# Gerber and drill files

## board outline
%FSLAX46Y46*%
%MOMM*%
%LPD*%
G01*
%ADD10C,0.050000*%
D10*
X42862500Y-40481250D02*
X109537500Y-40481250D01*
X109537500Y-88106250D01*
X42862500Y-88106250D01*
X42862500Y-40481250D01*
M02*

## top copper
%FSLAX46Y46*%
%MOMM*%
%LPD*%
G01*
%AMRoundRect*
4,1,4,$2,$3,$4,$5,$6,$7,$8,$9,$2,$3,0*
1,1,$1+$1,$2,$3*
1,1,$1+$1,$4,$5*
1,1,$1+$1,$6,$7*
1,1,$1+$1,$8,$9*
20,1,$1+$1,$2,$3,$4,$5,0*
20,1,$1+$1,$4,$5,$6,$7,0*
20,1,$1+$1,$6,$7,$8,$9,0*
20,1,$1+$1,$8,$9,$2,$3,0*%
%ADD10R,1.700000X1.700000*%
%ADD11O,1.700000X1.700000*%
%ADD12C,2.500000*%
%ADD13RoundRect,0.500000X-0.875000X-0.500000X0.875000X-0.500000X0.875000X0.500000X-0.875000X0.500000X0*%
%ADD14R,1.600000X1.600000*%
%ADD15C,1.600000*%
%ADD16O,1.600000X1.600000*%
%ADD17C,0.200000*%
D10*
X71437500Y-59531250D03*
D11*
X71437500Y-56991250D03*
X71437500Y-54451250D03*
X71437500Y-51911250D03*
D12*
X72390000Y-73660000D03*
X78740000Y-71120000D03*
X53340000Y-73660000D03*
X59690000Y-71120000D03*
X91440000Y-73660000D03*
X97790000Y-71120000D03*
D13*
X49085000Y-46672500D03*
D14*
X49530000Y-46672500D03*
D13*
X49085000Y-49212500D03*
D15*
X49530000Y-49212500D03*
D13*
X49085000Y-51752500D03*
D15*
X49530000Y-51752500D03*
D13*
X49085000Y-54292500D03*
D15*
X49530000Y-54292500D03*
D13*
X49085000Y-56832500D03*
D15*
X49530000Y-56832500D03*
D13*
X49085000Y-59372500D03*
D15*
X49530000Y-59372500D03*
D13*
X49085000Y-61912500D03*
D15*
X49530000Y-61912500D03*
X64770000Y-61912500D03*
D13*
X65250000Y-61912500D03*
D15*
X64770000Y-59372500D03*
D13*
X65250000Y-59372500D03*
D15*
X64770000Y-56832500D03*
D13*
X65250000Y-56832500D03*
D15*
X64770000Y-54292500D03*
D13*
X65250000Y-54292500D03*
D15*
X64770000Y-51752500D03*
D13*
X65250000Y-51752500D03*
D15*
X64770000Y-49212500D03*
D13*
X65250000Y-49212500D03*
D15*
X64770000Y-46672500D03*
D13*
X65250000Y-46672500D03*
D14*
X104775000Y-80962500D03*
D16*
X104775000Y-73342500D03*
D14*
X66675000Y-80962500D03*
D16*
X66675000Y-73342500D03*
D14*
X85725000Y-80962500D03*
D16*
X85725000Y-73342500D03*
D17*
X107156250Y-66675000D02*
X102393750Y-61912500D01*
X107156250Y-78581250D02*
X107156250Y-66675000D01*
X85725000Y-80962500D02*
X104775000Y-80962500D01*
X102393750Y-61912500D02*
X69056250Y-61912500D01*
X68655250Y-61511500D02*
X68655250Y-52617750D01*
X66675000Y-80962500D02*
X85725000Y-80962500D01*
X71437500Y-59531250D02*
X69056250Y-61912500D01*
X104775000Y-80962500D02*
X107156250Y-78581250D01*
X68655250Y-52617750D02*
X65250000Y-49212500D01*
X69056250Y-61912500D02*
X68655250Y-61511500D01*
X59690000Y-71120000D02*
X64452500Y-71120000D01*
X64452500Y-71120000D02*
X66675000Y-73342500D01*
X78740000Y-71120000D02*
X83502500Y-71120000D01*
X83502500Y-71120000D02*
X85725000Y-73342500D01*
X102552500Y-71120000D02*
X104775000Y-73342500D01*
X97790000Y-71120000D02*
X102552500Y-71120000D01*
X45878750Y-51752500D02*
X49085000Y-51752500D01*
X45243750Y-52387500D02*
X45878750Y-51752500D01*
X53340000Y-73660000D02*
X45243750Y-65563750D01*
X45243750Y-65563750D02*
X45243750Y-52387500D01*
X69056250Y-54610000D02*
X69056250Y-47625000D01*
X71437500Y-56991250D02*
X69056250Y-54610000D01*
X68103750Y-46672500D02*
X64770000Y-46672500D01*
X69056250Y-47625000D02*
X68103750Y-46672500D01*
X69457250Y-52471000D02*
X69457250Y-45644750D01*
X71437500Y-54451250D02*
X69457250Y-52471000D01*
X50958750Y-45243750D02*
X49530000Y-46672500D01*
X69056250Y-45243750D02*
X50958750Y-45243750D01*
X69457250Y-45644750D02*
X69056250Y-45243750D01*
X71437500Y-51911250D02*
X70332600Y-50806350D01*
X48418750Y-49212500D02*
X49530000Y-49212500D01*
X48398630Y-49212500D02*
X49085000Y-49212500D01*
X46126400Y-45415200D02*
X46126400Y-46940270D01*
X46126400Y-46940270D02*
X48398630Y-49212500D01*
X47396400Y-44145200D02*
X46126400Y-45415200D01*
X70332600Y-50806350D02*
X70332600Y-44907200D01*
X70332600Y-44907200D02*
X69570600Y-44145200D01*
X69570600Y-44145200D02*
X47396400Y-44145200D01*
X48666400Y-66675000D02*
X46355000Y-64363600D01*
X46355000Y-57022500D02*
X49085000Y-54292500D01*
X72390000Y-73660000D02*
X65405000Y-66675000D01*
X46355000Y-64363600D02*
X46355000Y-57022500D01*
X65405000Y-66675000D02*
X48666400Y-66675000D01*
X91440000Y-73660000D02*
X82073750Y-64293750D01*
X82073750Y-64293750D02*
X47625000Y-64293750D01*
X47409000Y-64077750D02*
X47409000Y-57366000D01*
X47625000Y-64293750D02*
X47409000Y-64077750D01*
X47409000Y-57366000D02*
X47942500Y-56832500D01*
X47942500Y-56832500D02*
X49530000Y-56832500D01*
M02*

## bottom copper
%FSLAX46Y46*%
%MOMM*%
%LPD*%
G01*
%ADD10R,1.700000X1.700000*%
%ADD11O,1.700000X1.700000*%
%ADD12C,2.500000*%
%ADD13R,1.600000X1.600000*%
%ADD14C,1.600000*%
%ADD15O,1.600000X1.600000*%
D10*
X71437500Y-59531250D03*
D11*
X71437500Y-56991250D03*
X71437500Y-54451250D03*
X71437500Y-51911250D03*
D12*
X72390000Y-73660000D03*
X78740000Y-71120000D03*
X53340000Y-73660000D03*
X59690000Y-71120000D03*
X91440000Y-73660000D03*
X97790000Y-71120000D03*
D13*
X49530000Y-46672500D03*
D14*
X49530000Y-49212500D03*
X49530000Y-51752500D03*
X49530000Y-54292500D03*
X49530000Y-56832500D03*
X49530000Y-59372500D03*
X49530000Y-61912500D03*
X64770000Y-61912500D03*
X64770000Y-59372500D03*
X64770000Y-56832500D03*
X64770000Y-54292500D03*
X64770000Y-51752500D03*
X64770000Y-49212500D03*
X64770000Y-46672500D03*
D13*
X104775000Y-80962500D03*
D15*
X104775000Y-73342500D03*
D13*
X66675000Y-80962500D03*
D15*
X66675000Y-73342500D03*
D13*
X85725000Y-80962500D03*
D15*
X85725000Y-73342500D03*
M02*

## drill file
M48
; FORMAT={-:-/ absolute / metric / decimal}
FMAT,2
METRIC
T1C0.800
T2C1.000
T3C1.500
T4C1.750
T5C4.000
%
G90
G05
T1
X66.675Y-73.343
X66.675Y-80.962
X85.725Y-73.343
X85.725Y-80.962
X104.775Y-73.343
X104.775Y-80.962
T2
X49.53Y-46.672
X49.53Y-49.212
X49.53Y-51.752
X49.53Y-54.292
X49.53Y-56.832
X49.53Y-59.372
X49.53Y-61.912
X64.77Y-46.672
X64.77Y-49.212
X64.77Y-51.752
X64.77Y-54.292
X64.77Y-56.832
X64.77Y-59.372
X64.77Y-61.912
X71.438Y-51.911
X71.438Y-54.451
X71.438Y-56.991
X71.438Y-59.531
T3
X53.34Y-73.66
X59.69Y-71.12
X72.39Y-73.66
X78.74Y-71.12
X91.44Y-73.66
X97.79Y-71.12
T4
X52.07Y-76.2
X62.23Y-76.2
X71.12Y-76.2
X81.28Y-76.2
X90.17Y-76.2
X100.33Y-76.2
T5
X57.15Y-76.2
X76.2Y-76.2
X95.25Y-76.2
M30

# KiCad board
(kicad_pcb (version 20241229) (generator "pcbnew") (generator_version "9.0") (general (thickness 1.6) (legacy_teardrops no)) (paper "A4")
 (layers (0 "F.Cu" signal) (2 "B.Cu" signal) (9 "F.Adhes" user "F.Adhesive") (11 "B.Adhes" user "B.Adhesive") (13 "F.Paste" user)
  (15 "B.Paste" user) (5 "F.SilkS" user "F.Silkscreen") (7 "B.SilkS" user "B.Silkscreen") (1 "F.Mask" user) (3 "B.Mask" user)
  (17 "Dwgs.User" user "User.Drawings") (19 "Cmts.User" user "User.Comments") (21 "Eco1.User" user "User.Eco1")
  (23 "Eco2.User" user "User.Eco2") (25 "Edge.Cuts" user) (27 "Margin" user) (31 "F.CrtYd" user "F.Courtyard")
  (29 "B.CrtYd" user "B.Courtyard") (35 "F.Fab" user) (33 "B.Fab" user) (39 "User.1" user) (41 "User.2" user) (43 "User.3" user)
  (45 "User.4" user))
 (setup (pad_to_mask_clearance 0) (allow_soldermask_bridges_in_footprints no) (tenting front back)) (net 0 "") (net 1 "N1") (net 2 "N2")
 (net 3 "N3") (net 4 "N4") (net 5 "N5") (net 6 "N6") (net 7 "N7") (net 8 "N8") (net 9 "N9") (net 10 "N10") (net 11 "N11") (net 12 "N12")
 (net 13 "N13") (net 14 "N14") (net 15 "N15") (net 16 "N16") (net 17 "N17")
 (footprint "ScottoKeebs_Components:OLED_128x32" (layer "F.Cu") (at 69.8375 49.73125)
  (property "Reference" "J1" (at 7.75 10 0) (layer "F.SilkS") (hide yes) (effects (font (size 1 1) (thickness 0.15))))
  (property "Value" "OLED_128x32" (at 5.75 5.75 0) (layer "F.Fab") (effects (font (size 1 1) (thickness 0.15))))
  (pad "1" thru_hole rect (at 1.6 9.8 180) (size 1.7 1.7) (drill 1) (layers "*.Cu" "*.Mask") (remove_unused_layers no) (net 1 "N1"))
  (pad "2" thru_hole oval (at 1.6 7.26 180) (size 1.7 1.7) (drill 1) (layers "*.Cu" "*.Mask") (remove_unused_layers no) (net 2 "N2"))
  (pad "3" thru_hole oval (at 1.6 4.72 180) (size 1.7 1.7) (drill 1) (layers "*.Cu" "*.Mask") (remove_unused_layers no) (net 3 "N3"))
  (pad "4" thru_hole oval (at 1.6 2.18 180) (size 1.7 1.7) (drill 1) (layers "*.Cu" "*.Mask") (remove_unused_layers no) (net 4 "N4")))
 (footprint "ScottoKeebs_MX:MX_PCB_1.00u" (layer "F.Cu") (at 76.2 76.2)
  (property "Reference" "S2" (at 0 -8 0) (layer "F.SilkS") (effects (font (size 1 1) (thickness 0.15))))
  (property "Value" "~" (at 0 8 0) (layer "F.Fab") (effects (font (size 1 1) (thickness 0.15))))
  (pad "" np_thru_hole circle (at -5.08 0) (size 1.75 1.75) (drill 1.75) (layers "*.Cu" "*.Mask"))
  (pad "" np_thru_hole circle (at 0 0) (size 4 4) (drill 4) (layers "*.Cu" "*.Mask"))
  (pad "" np_thru_hole circle (at 5.08 0) (size 1.75 1.75) (drill 1.75) (layers "*.Cu" "*.Mask"))
  (pad "1" thru_hole circle (at -3.81 -2.54) (size 2.5 2.5) (drill 1.5) (layers "*.Cu" "*.Mask") (remove_unused_layers no) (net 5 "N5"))
  (pad "2" thru_hole circle (at 2.54 -5.08) (size 2.5 2.5) (drill 1.5) (layers "*.Cu" "*.Mask") (remove_unused_layers no) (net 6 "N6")))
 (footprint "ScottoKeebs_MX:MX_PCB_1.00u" (layer "F.Cu") (at 57.15 76.2)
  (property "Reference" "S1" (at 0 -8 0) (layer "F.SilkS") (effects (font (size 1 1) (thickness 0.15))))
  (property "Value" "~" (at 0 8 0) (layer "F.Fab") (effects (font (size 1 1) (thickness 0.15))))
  (pad "" np_thru_hole circle (at -5.08 0) (size 1.75 1.75) (drill 1.75) (layers "*.Cu" "*.Mask"))
  (pad "" np_thru_hole circle (at 0 0) (size 4 4) (drill 4) (layers "*.Cu" "*.Mask"))
  (pad "" np_thru_hole circle (at 5.08 0) (size 1.75 1.75) (drill 1.75) (layers "*.Cu" "*.Mask"))
  (pad "1" thru_hole circle (at -3.81 -2.54) (size 2.5 2.5) (drill 1.5) (layers "*.Cu" "*.Mask") (remove_unused_layers no) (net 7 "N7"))
  (pad "2" thru_hole circle (at 2.54 -5.08) (size 2.5 2.5) (drill 1.5) (layers "*.Cu" "*.Mask") (remove_unused_layers no) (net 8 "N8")))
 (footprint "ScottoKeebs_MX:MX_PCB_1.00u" (layer "F.Cu") (at 95.25 76.2)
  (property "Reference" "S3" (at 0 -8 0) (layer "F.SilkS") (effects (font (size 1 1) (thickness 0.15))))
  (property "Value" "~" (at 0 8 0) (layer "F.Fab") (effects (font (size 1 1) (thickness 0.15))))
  (pad "" np_thru_hole circle (at -5.08 0) (size 1.75 1.75) (drill 1.75) (layers "*.Cu" "*.Mask"))
  (pad "" np_thru_hole circle (at 0 0) (size 4 4) (drill 4) (layers "*.Cu" "*.Mask"))
  (pad "" np_thru_hole circle (at 5.08 0) (size 1.75 1.75) (drill 1.75) (layers "*.Cu" "*.Mask"))
  (pad "1" thru_hole circle (at -3.81 -2.54) (size 2.5 2.5) (drill 1.5) (layers "*.Cu" "*.Mask") (remove_unused_layers no) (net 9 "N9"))
  (pad "2" thru_hole circle (at 2.54 -5.08) (size 2.5 2.5) (drill 1.5) (layers "*.Cu" "*.Mask") (remove_unused_layers no) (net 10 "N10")))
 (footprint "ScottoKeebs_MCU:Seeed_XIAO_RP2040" (layer "F.Cu") (at 57.15 54.2925)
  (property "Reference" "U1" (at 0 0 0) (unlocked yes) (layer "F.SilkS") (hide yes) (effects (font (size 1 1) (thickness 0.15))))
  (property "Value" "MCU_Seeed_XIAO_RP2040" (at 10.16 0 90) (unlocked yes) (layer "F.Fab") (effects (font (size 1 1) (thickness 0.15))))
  (pad "1" smd roundrect (at -8.065 -7.62) (size 2.75 2) (layers "F.Cu" "F.Mask" "F.Paste") (roundrect_rratio 0.25) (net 3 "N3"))
  (pad "1" thru_hole rect (at -7.62 -7.62 90) (size 1.6 1.6) (drill 1) (layers "*.Cu" "*.Mask") (remove_unused_layers no) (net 3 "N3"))
  (pad "2" smd roundrect (at -8.065 -5.08) (size 2.75 2) (layers "F.Cu" "F.Mask" "F.Paste") (roundrect_rratio 0.25) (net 4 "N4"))
  (pad "2" thru_hole circle (at -7.62 -5.08 90) (size 1.6 1.6) (drill 1) (layers "*.Cu" "*.Mask") (remove_unused_layers no) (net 4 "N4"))
  (pad "3" smd roundrect (at -8.065 -2.54) (size 2.75 2) (layers "F.Cu" "F.Mask" "F.Paste") (roundrect_rratio 0.25) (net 7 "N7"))
  (pad "3" thru_hole circle (at -7.62 -2.54 90) (size 1.6 1.6) (drill 1) (layers "*.Cu" "*.Mask") (remove_unused_layers no) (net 7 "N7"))
  (pad "4" smd roundrect (at -8.065 0) (size 2.75 2) (layers "F.Cu" "F.Mask" "F.Paste") (roundrect_rratio 0.25) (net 5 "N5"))
  (pad "4" thru_hole circle (at -7.62 0 90) (size 1.6 1.6) (drill 1) (layers "*.Cu" "*.Mask") (remove_unused_layers no) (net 5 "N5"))
  (pad "5" smd roundrect (at -8.065 2.54) (size 2.75 2) (layers "F.Cu" "F.Mask" "F.Paste") (roundrect_rratio 0.25) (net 9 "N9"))
  (pad "5" thru_hole circle (at -7.62 2.54 90) (size 1.6 1.6) (drill 1) (layers "*.Cu" "*.Mask") (remove_unused_layers no) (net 9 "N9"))
  (pad "6" smd roundrect (at -8.065 5.08) (size 2.75 2) (layers "F.Cu" "F.Mask" "F.Paste") (roundrect_rratio 0.25) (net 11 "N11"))
  (pad "6" thru_hole circle (at -7.62 5.08 90) (size 1.6 1.6) (drill 1) (layers "*.Cu" "*.Mask") (remove_unused_layers no) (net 11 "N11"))
  (pad "7" smd roundrect (at -8.065 7.62) (size 2.75 2) (layers "F.Cu" "F.Mask" "F.Paste") (roundrect_rratio 0.25) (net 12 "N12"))
  (pad "7" thru_hole circle (at -7.62 7.62 90) (size 1.6 1.6) (drill 1) (layers "*.Cu" "*.Mask") (remove_unused_layers no) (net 12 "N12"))
  (pad "8" thru_hole circle (at 7.62 7.62 90) (size 1.6 1.6) (drill 1) (layers "*.Cu" "*.Mask") (remove_unused_layers no) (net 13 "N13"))
  (pad "8" smd roundrect (at 8.1 7.62) (size 2.75 2) (layers "F.Cu" "F.Mask" "F.Paste") (roundrect_rratio 0.25) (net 13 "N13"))
  (pad "9" thru_hole circle (at 7.62 5.08 90) (size 1.6 1.6) (drill 1) (layers "*.Cu" "*.Mask") (remove_unused_layers no) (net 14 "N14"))
  (pad "9" smd roundrect (at 8.1 5.08) (size 2.75 2) (layers "F.Cu" "F.Mask" "F.Paste") (roundrect_rratio 0.25) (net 14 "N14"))
  (pad "10" thru_hole circle (at 7.62 2.54 90) (size 1.6 1.6) (drill 1) (layers "*.Cu" "*.Mask") (remove_unused_layers no) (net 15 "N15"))
  (pad "10" smd roundrect (at 8.1 2.54) (size 2.75 2) (layers "F.Cu" "F.Mask" "F.Paste") (roundrect_rratio 0.25) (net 15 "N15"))
  (pad "11" thru_hole circle (at 7.62 0 90) (size 1.6 1.6) (drill 1) (layers "*.Cu" "*.Mask") (remove_unused_layers no) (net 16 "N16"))
  (pad "11" smd roundrect (at 8.1 0) (size 2.75 2) (layers "F.Cu" "F.Mask" "F.Paste") (roundrect_rratio 0.25) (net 16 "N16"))
  (pad "12" thru_hole circle (at 7.62 -2.54 90) (size 1.6 1.6) (drill 1) (layers "*.Cu" "*.Mask") (remove_unused_layers no) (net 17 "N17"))
  (pad "12" smd roundrect (at 8.1 -2.54) (size 2.75 2) (layers "F.Cu" "F.Mask" "F.Paste") (roundrect_rratio 0.25) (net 17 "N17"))
  (pad "13" thru_hole circle (at 7.62 -5.08 90) (size 1.6 1.6) (drill 1) (layers "*.Cu" "*.Mask") (remove_unused_layers no) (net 1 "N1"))
  (pad "13" smd roundrect (at 8.1 -5.08) (size 2.75 2) (layers "F.Cu" "F.Mask" "F.Paste") (roundrect_rratio 0.25) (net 1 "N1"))
  (pad "14" thru_hole circle (at 7.62 -7.62 90) (size 1.6 1.6) (drill 1) (layers "*.Cu" "*.Mask") (remove_unused_layers no) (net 2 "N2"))
  (pad "14" smd roundrect (at 8.1 -7.62) (size 2.75 2) (layers "F.Cu" "F.Mask" "F.Paste") (roundrect_rratio 0.25) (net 2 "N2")))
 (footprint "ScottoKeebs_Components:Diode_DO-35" (layer "B.Cu") (at 104.775 80.9625 90)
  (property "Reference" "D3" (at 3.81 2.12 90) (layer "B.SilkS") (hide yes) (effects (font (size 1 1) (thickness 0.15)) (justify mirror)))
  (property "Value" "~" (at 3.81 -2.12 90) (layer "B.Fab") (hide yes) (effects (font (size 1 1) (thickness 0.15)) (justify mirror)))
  (pad "1" thru_hole rect (at 0 0 90) (size 1.6 1.6) (drill 0.8) (layers "*.Cu" "*.Mask") (remove_unused_layers no) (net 1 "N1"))
  (pad "2" thru_hole oval (at 7.62 0 90) (size 1.6 1.6) (drill 0.8) (layers "*.Cu" "*.Mask") (remove_unused_layers no) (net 10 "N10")))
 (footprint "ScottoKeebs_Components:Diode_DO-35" (layer "B.Cu") (at 66.675 80.9625 90)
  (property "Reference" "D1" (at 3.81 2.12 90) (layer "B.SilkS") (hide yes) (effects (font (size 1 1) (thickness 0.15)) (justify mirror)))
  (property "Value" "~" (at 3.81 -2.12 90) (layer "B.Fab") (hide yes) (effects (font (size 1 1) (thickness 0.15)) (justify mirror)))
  (pad "1" thru_hole rect (at 0 0 90) (size 1.6 1.6) (drill 0.8) (layers "*.Cu" "*.Mask") (remove_unused_layers no) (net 1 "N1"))
  (pad "2" thru_hole oval (at 7.62 0 90) (size 1.6 1.6) (drill 0.8) (layers "*.Cu" "*.Mask") (remove_unused_layers no) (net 8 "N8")))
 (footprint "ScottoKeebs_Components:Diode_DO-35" (layer "B.Cu") (at 85.725 80.9625 90)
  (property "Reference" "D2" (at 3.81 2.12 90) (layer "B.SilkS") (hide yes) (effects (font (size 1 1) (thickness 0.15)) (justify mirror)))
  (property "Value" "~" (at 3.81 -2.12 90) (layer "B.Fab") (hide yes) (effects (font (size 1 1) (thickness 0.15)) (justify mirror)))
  (pad "1" thru_hole rect (at 0 0 90) (size 1.6 1.6) (drill 0.8) (layers "*.Cu" "*.Mask") (remove_unused_layers no) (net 1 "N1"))
  (pad "2" thru_hole oval (at 7.62 0 90) (size 1.6 1.6) (drill 0.8) (layers "*.Cu" "*.Mask") (remove_unused_layers no) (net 6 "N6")))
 (gr_rect (start 42.8625 40.48125) (end 109.5375 88.10625) (stroke (width 0.05) (type default)) (fill no) (layer "Edge.Cuts"))
 (segment (start 107.15625 66.675) (end 102.39375 61.9125) (width 0.2) (layer "F.Cu") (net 1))
 (segment (start 107.15625 78.58125) (end 107.15625 66.675) (width 0.2) (layer "F.Cu") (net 1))
 (segment (start 85.725 80.9625) (end 104.775 80.9625) (width 0.2) (layer "F.Cu") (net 1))
 (segment (start 102.39375 61.9125) (end 69.05625 61.9125) (width 0.2) (layer "F.Cu") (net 1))
 (segment (start 68.65525 61.5115) (end 68.65525 52.61775) (width 0.2) (layer "F.Cu") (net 1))
 (segment (start 66.675 80.9625) (end 85.725 80.9625) (width 0.2) (layer "F.Cu") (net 1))
 (segment (start 71.4375 59.53125) (end 69.05625 61.9125) (width 0.2) (layer "F.Cu") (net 1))
 (segment (start 104.775 80.9625) (end 107.15625 78.58125) (width 0.2) (layer "F.Cu") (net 1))
 (segment (start 68.65525 52.61775) (end 65.25 49.2125) (width 0.2) (layer "F.Cu") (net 1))
 (segment (start 69.05625 61.9125) (end 68.65525 61.5115) (width 0.2) (layer "F.Cu") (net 1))
 (segment (start 59.69 71.12) (end 64.4525 71.12) (width 0.2) (layer "F.Cu") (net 8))
 (segment (start 64.4525 71.12) (end 66.675 73.3425) (width 0.2) (layer "F.Cu") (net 8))
 (segment (start 78.74 71.12) (end 83.5025 71.12) (width 0.2) (layer "F.Cu") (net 6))
 (segment (start 83.5025 71.12) (end 85.725 73.3425) (width 0.2) (layer "F.Cu") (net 6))
 (segment (start 102.5525 71.12) (end 104.775 73.3425) (width 0.2) (layer "F.Cu") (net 10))
 (segment (start 97.79 71.12) (end 102.5525 71.12) (width 0.2) (layer "F.Cu") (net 10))
 (segment (start 45.87875 51.7525) (end 49.085 51.7525) (width 0.2) (layer "F.Cu") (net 7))
 (segment (start 45.24375 52.3875) (end 45.87875 51.7525) (width 0.2) (layer "F.Cu") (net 7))
 (segment (start 53.34 73.66) (end 45.24375 65.56375) (width 0.2) (layer "F.Cu") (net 7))
 (segment (start 45.24375 65.56375) (end 45.24375 52.3875) (width 0.2) (layer "F.Cu") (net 7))
 (segment (start 69.05625 54.61) (end 69.05625 47.625) (width 0.2) (layer "F.Cu") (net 2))
 (segment (start 71.4375 56.99125) (end 69.05625 54.61) (width 0.2) (layer "F.Cu") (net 2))
 (segment (start 68.10375 46.6725) (end 64.77 46.6725) (width 0.2) (layer "F.Cu") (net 2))
 (segment (start 69.05625 47.625) (end 68.10375 46.6725) (width 0.2) (layer "F.Cu") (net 2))
 (segment (start 69.45725 52.471) (end 69.45725 45.64475) (width 0.2) (layer "F.Cu") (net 3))
 (segment (start 71.4375 54.45125) (end 69.45725 52.471) (width 0.2) (layer "F.Cu") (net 3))
 (segment (start 50.95875 45.24375) (end 49.53 46.6725) (width 0.2) (layer "F.Cu") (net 3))
 (segment (start 69.05625 45.24375) (end 50.95875 45.24375) (width 0.2) (layer "F.Cu") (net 3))
 (segment (start 69.45725 45.64475) (end 69.05625 45.24375) (width 0.2) (layer "F.Cu") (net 3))
 (segment (start 71.4375 51.91125) (end 70.3326 50.80635) (width 0.2) (layer "F.Cu") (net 4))
 (segment (start 48.41875 49.2125) (end 49.53 49.2125) (width 0.2) (layer "F.Cu") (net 4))
 (segment (start 48.39863 49.2125) (end 49.085 49.2125) (width 0.2) (layer "F.Cu") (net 4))
 (segment (start 46.1264 45.4152) (end 46.1264 46.94027) (width 0.2) (layer "F.Cu") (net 4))
 (segment (start 46.1264 46.94027) (end 48.39863 49.2125) (width 0.2) (layer "F.Cu") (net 4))
 (segment (start 47.3964 44.1452) (end 46.1264 45.4152) (width 0.2) (layer "F.Cu") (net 4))
 (segment (start 70.3326 50.80635) (end 70.3326 44.9072) (width 0.2) (layer "F.Cu") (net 4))
 (segment (start 70.3326 44.9072) (end 69.5706 44.1452) (width 0.2) (layer "F.Cu") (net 4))
 (segment (start 69.5706 44.1452) (end 47.3964 44.1452) (width 0.2) (layer "F.Cu") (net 4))
 (segment (start 48.6664 66.675) (end 46.355 64.3636) (width 0.2) (layer "F.Cu") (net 5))
 (segment (start 46.355 57.0225) (end 49.085 54.2925) (width 0.2) (layer "F.Cu") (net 5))
 (segment (start 72.39 73.66) (end 65.405 66.675) (width 0.2) (layer "F.Cu") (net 5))
 (segment (start 46.355 64.3636) (end 46.355 57.0225) (width 0.2) (layer "F.Cu") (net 5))
 (segment (start 65.405 66.675) (end 48.6664 66.675) (width 0.2) (layer "F.Cu") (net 5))
 (segment (start 91.44 73.66) (end 82.07375 64.29375) (width 0.2) (layer "F.Cu") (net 9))
 (segment (start 82.07375 64.29375) (end 47.625 64.29375) (width 0.2) (layer "F.Cu") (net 9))
 (segment (start 47.409 64.07775) (end 47.409 57.366) (width 0.2) (layer "F.Cu") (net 9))
 (segment (start 47.625 64.29375) (end 47.409 64.07775) (width 0.2) (layer "F.Cu") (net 9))
 (segment (start 47.409 57.366) (end 47.9425 56.8325) (width 0.2) (layer "F.Cu") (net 9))
 (segment (start 47.9425 56.8325) (end 49.53 56.8325) (width 0.2) (layer "F.Cu") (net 9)))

